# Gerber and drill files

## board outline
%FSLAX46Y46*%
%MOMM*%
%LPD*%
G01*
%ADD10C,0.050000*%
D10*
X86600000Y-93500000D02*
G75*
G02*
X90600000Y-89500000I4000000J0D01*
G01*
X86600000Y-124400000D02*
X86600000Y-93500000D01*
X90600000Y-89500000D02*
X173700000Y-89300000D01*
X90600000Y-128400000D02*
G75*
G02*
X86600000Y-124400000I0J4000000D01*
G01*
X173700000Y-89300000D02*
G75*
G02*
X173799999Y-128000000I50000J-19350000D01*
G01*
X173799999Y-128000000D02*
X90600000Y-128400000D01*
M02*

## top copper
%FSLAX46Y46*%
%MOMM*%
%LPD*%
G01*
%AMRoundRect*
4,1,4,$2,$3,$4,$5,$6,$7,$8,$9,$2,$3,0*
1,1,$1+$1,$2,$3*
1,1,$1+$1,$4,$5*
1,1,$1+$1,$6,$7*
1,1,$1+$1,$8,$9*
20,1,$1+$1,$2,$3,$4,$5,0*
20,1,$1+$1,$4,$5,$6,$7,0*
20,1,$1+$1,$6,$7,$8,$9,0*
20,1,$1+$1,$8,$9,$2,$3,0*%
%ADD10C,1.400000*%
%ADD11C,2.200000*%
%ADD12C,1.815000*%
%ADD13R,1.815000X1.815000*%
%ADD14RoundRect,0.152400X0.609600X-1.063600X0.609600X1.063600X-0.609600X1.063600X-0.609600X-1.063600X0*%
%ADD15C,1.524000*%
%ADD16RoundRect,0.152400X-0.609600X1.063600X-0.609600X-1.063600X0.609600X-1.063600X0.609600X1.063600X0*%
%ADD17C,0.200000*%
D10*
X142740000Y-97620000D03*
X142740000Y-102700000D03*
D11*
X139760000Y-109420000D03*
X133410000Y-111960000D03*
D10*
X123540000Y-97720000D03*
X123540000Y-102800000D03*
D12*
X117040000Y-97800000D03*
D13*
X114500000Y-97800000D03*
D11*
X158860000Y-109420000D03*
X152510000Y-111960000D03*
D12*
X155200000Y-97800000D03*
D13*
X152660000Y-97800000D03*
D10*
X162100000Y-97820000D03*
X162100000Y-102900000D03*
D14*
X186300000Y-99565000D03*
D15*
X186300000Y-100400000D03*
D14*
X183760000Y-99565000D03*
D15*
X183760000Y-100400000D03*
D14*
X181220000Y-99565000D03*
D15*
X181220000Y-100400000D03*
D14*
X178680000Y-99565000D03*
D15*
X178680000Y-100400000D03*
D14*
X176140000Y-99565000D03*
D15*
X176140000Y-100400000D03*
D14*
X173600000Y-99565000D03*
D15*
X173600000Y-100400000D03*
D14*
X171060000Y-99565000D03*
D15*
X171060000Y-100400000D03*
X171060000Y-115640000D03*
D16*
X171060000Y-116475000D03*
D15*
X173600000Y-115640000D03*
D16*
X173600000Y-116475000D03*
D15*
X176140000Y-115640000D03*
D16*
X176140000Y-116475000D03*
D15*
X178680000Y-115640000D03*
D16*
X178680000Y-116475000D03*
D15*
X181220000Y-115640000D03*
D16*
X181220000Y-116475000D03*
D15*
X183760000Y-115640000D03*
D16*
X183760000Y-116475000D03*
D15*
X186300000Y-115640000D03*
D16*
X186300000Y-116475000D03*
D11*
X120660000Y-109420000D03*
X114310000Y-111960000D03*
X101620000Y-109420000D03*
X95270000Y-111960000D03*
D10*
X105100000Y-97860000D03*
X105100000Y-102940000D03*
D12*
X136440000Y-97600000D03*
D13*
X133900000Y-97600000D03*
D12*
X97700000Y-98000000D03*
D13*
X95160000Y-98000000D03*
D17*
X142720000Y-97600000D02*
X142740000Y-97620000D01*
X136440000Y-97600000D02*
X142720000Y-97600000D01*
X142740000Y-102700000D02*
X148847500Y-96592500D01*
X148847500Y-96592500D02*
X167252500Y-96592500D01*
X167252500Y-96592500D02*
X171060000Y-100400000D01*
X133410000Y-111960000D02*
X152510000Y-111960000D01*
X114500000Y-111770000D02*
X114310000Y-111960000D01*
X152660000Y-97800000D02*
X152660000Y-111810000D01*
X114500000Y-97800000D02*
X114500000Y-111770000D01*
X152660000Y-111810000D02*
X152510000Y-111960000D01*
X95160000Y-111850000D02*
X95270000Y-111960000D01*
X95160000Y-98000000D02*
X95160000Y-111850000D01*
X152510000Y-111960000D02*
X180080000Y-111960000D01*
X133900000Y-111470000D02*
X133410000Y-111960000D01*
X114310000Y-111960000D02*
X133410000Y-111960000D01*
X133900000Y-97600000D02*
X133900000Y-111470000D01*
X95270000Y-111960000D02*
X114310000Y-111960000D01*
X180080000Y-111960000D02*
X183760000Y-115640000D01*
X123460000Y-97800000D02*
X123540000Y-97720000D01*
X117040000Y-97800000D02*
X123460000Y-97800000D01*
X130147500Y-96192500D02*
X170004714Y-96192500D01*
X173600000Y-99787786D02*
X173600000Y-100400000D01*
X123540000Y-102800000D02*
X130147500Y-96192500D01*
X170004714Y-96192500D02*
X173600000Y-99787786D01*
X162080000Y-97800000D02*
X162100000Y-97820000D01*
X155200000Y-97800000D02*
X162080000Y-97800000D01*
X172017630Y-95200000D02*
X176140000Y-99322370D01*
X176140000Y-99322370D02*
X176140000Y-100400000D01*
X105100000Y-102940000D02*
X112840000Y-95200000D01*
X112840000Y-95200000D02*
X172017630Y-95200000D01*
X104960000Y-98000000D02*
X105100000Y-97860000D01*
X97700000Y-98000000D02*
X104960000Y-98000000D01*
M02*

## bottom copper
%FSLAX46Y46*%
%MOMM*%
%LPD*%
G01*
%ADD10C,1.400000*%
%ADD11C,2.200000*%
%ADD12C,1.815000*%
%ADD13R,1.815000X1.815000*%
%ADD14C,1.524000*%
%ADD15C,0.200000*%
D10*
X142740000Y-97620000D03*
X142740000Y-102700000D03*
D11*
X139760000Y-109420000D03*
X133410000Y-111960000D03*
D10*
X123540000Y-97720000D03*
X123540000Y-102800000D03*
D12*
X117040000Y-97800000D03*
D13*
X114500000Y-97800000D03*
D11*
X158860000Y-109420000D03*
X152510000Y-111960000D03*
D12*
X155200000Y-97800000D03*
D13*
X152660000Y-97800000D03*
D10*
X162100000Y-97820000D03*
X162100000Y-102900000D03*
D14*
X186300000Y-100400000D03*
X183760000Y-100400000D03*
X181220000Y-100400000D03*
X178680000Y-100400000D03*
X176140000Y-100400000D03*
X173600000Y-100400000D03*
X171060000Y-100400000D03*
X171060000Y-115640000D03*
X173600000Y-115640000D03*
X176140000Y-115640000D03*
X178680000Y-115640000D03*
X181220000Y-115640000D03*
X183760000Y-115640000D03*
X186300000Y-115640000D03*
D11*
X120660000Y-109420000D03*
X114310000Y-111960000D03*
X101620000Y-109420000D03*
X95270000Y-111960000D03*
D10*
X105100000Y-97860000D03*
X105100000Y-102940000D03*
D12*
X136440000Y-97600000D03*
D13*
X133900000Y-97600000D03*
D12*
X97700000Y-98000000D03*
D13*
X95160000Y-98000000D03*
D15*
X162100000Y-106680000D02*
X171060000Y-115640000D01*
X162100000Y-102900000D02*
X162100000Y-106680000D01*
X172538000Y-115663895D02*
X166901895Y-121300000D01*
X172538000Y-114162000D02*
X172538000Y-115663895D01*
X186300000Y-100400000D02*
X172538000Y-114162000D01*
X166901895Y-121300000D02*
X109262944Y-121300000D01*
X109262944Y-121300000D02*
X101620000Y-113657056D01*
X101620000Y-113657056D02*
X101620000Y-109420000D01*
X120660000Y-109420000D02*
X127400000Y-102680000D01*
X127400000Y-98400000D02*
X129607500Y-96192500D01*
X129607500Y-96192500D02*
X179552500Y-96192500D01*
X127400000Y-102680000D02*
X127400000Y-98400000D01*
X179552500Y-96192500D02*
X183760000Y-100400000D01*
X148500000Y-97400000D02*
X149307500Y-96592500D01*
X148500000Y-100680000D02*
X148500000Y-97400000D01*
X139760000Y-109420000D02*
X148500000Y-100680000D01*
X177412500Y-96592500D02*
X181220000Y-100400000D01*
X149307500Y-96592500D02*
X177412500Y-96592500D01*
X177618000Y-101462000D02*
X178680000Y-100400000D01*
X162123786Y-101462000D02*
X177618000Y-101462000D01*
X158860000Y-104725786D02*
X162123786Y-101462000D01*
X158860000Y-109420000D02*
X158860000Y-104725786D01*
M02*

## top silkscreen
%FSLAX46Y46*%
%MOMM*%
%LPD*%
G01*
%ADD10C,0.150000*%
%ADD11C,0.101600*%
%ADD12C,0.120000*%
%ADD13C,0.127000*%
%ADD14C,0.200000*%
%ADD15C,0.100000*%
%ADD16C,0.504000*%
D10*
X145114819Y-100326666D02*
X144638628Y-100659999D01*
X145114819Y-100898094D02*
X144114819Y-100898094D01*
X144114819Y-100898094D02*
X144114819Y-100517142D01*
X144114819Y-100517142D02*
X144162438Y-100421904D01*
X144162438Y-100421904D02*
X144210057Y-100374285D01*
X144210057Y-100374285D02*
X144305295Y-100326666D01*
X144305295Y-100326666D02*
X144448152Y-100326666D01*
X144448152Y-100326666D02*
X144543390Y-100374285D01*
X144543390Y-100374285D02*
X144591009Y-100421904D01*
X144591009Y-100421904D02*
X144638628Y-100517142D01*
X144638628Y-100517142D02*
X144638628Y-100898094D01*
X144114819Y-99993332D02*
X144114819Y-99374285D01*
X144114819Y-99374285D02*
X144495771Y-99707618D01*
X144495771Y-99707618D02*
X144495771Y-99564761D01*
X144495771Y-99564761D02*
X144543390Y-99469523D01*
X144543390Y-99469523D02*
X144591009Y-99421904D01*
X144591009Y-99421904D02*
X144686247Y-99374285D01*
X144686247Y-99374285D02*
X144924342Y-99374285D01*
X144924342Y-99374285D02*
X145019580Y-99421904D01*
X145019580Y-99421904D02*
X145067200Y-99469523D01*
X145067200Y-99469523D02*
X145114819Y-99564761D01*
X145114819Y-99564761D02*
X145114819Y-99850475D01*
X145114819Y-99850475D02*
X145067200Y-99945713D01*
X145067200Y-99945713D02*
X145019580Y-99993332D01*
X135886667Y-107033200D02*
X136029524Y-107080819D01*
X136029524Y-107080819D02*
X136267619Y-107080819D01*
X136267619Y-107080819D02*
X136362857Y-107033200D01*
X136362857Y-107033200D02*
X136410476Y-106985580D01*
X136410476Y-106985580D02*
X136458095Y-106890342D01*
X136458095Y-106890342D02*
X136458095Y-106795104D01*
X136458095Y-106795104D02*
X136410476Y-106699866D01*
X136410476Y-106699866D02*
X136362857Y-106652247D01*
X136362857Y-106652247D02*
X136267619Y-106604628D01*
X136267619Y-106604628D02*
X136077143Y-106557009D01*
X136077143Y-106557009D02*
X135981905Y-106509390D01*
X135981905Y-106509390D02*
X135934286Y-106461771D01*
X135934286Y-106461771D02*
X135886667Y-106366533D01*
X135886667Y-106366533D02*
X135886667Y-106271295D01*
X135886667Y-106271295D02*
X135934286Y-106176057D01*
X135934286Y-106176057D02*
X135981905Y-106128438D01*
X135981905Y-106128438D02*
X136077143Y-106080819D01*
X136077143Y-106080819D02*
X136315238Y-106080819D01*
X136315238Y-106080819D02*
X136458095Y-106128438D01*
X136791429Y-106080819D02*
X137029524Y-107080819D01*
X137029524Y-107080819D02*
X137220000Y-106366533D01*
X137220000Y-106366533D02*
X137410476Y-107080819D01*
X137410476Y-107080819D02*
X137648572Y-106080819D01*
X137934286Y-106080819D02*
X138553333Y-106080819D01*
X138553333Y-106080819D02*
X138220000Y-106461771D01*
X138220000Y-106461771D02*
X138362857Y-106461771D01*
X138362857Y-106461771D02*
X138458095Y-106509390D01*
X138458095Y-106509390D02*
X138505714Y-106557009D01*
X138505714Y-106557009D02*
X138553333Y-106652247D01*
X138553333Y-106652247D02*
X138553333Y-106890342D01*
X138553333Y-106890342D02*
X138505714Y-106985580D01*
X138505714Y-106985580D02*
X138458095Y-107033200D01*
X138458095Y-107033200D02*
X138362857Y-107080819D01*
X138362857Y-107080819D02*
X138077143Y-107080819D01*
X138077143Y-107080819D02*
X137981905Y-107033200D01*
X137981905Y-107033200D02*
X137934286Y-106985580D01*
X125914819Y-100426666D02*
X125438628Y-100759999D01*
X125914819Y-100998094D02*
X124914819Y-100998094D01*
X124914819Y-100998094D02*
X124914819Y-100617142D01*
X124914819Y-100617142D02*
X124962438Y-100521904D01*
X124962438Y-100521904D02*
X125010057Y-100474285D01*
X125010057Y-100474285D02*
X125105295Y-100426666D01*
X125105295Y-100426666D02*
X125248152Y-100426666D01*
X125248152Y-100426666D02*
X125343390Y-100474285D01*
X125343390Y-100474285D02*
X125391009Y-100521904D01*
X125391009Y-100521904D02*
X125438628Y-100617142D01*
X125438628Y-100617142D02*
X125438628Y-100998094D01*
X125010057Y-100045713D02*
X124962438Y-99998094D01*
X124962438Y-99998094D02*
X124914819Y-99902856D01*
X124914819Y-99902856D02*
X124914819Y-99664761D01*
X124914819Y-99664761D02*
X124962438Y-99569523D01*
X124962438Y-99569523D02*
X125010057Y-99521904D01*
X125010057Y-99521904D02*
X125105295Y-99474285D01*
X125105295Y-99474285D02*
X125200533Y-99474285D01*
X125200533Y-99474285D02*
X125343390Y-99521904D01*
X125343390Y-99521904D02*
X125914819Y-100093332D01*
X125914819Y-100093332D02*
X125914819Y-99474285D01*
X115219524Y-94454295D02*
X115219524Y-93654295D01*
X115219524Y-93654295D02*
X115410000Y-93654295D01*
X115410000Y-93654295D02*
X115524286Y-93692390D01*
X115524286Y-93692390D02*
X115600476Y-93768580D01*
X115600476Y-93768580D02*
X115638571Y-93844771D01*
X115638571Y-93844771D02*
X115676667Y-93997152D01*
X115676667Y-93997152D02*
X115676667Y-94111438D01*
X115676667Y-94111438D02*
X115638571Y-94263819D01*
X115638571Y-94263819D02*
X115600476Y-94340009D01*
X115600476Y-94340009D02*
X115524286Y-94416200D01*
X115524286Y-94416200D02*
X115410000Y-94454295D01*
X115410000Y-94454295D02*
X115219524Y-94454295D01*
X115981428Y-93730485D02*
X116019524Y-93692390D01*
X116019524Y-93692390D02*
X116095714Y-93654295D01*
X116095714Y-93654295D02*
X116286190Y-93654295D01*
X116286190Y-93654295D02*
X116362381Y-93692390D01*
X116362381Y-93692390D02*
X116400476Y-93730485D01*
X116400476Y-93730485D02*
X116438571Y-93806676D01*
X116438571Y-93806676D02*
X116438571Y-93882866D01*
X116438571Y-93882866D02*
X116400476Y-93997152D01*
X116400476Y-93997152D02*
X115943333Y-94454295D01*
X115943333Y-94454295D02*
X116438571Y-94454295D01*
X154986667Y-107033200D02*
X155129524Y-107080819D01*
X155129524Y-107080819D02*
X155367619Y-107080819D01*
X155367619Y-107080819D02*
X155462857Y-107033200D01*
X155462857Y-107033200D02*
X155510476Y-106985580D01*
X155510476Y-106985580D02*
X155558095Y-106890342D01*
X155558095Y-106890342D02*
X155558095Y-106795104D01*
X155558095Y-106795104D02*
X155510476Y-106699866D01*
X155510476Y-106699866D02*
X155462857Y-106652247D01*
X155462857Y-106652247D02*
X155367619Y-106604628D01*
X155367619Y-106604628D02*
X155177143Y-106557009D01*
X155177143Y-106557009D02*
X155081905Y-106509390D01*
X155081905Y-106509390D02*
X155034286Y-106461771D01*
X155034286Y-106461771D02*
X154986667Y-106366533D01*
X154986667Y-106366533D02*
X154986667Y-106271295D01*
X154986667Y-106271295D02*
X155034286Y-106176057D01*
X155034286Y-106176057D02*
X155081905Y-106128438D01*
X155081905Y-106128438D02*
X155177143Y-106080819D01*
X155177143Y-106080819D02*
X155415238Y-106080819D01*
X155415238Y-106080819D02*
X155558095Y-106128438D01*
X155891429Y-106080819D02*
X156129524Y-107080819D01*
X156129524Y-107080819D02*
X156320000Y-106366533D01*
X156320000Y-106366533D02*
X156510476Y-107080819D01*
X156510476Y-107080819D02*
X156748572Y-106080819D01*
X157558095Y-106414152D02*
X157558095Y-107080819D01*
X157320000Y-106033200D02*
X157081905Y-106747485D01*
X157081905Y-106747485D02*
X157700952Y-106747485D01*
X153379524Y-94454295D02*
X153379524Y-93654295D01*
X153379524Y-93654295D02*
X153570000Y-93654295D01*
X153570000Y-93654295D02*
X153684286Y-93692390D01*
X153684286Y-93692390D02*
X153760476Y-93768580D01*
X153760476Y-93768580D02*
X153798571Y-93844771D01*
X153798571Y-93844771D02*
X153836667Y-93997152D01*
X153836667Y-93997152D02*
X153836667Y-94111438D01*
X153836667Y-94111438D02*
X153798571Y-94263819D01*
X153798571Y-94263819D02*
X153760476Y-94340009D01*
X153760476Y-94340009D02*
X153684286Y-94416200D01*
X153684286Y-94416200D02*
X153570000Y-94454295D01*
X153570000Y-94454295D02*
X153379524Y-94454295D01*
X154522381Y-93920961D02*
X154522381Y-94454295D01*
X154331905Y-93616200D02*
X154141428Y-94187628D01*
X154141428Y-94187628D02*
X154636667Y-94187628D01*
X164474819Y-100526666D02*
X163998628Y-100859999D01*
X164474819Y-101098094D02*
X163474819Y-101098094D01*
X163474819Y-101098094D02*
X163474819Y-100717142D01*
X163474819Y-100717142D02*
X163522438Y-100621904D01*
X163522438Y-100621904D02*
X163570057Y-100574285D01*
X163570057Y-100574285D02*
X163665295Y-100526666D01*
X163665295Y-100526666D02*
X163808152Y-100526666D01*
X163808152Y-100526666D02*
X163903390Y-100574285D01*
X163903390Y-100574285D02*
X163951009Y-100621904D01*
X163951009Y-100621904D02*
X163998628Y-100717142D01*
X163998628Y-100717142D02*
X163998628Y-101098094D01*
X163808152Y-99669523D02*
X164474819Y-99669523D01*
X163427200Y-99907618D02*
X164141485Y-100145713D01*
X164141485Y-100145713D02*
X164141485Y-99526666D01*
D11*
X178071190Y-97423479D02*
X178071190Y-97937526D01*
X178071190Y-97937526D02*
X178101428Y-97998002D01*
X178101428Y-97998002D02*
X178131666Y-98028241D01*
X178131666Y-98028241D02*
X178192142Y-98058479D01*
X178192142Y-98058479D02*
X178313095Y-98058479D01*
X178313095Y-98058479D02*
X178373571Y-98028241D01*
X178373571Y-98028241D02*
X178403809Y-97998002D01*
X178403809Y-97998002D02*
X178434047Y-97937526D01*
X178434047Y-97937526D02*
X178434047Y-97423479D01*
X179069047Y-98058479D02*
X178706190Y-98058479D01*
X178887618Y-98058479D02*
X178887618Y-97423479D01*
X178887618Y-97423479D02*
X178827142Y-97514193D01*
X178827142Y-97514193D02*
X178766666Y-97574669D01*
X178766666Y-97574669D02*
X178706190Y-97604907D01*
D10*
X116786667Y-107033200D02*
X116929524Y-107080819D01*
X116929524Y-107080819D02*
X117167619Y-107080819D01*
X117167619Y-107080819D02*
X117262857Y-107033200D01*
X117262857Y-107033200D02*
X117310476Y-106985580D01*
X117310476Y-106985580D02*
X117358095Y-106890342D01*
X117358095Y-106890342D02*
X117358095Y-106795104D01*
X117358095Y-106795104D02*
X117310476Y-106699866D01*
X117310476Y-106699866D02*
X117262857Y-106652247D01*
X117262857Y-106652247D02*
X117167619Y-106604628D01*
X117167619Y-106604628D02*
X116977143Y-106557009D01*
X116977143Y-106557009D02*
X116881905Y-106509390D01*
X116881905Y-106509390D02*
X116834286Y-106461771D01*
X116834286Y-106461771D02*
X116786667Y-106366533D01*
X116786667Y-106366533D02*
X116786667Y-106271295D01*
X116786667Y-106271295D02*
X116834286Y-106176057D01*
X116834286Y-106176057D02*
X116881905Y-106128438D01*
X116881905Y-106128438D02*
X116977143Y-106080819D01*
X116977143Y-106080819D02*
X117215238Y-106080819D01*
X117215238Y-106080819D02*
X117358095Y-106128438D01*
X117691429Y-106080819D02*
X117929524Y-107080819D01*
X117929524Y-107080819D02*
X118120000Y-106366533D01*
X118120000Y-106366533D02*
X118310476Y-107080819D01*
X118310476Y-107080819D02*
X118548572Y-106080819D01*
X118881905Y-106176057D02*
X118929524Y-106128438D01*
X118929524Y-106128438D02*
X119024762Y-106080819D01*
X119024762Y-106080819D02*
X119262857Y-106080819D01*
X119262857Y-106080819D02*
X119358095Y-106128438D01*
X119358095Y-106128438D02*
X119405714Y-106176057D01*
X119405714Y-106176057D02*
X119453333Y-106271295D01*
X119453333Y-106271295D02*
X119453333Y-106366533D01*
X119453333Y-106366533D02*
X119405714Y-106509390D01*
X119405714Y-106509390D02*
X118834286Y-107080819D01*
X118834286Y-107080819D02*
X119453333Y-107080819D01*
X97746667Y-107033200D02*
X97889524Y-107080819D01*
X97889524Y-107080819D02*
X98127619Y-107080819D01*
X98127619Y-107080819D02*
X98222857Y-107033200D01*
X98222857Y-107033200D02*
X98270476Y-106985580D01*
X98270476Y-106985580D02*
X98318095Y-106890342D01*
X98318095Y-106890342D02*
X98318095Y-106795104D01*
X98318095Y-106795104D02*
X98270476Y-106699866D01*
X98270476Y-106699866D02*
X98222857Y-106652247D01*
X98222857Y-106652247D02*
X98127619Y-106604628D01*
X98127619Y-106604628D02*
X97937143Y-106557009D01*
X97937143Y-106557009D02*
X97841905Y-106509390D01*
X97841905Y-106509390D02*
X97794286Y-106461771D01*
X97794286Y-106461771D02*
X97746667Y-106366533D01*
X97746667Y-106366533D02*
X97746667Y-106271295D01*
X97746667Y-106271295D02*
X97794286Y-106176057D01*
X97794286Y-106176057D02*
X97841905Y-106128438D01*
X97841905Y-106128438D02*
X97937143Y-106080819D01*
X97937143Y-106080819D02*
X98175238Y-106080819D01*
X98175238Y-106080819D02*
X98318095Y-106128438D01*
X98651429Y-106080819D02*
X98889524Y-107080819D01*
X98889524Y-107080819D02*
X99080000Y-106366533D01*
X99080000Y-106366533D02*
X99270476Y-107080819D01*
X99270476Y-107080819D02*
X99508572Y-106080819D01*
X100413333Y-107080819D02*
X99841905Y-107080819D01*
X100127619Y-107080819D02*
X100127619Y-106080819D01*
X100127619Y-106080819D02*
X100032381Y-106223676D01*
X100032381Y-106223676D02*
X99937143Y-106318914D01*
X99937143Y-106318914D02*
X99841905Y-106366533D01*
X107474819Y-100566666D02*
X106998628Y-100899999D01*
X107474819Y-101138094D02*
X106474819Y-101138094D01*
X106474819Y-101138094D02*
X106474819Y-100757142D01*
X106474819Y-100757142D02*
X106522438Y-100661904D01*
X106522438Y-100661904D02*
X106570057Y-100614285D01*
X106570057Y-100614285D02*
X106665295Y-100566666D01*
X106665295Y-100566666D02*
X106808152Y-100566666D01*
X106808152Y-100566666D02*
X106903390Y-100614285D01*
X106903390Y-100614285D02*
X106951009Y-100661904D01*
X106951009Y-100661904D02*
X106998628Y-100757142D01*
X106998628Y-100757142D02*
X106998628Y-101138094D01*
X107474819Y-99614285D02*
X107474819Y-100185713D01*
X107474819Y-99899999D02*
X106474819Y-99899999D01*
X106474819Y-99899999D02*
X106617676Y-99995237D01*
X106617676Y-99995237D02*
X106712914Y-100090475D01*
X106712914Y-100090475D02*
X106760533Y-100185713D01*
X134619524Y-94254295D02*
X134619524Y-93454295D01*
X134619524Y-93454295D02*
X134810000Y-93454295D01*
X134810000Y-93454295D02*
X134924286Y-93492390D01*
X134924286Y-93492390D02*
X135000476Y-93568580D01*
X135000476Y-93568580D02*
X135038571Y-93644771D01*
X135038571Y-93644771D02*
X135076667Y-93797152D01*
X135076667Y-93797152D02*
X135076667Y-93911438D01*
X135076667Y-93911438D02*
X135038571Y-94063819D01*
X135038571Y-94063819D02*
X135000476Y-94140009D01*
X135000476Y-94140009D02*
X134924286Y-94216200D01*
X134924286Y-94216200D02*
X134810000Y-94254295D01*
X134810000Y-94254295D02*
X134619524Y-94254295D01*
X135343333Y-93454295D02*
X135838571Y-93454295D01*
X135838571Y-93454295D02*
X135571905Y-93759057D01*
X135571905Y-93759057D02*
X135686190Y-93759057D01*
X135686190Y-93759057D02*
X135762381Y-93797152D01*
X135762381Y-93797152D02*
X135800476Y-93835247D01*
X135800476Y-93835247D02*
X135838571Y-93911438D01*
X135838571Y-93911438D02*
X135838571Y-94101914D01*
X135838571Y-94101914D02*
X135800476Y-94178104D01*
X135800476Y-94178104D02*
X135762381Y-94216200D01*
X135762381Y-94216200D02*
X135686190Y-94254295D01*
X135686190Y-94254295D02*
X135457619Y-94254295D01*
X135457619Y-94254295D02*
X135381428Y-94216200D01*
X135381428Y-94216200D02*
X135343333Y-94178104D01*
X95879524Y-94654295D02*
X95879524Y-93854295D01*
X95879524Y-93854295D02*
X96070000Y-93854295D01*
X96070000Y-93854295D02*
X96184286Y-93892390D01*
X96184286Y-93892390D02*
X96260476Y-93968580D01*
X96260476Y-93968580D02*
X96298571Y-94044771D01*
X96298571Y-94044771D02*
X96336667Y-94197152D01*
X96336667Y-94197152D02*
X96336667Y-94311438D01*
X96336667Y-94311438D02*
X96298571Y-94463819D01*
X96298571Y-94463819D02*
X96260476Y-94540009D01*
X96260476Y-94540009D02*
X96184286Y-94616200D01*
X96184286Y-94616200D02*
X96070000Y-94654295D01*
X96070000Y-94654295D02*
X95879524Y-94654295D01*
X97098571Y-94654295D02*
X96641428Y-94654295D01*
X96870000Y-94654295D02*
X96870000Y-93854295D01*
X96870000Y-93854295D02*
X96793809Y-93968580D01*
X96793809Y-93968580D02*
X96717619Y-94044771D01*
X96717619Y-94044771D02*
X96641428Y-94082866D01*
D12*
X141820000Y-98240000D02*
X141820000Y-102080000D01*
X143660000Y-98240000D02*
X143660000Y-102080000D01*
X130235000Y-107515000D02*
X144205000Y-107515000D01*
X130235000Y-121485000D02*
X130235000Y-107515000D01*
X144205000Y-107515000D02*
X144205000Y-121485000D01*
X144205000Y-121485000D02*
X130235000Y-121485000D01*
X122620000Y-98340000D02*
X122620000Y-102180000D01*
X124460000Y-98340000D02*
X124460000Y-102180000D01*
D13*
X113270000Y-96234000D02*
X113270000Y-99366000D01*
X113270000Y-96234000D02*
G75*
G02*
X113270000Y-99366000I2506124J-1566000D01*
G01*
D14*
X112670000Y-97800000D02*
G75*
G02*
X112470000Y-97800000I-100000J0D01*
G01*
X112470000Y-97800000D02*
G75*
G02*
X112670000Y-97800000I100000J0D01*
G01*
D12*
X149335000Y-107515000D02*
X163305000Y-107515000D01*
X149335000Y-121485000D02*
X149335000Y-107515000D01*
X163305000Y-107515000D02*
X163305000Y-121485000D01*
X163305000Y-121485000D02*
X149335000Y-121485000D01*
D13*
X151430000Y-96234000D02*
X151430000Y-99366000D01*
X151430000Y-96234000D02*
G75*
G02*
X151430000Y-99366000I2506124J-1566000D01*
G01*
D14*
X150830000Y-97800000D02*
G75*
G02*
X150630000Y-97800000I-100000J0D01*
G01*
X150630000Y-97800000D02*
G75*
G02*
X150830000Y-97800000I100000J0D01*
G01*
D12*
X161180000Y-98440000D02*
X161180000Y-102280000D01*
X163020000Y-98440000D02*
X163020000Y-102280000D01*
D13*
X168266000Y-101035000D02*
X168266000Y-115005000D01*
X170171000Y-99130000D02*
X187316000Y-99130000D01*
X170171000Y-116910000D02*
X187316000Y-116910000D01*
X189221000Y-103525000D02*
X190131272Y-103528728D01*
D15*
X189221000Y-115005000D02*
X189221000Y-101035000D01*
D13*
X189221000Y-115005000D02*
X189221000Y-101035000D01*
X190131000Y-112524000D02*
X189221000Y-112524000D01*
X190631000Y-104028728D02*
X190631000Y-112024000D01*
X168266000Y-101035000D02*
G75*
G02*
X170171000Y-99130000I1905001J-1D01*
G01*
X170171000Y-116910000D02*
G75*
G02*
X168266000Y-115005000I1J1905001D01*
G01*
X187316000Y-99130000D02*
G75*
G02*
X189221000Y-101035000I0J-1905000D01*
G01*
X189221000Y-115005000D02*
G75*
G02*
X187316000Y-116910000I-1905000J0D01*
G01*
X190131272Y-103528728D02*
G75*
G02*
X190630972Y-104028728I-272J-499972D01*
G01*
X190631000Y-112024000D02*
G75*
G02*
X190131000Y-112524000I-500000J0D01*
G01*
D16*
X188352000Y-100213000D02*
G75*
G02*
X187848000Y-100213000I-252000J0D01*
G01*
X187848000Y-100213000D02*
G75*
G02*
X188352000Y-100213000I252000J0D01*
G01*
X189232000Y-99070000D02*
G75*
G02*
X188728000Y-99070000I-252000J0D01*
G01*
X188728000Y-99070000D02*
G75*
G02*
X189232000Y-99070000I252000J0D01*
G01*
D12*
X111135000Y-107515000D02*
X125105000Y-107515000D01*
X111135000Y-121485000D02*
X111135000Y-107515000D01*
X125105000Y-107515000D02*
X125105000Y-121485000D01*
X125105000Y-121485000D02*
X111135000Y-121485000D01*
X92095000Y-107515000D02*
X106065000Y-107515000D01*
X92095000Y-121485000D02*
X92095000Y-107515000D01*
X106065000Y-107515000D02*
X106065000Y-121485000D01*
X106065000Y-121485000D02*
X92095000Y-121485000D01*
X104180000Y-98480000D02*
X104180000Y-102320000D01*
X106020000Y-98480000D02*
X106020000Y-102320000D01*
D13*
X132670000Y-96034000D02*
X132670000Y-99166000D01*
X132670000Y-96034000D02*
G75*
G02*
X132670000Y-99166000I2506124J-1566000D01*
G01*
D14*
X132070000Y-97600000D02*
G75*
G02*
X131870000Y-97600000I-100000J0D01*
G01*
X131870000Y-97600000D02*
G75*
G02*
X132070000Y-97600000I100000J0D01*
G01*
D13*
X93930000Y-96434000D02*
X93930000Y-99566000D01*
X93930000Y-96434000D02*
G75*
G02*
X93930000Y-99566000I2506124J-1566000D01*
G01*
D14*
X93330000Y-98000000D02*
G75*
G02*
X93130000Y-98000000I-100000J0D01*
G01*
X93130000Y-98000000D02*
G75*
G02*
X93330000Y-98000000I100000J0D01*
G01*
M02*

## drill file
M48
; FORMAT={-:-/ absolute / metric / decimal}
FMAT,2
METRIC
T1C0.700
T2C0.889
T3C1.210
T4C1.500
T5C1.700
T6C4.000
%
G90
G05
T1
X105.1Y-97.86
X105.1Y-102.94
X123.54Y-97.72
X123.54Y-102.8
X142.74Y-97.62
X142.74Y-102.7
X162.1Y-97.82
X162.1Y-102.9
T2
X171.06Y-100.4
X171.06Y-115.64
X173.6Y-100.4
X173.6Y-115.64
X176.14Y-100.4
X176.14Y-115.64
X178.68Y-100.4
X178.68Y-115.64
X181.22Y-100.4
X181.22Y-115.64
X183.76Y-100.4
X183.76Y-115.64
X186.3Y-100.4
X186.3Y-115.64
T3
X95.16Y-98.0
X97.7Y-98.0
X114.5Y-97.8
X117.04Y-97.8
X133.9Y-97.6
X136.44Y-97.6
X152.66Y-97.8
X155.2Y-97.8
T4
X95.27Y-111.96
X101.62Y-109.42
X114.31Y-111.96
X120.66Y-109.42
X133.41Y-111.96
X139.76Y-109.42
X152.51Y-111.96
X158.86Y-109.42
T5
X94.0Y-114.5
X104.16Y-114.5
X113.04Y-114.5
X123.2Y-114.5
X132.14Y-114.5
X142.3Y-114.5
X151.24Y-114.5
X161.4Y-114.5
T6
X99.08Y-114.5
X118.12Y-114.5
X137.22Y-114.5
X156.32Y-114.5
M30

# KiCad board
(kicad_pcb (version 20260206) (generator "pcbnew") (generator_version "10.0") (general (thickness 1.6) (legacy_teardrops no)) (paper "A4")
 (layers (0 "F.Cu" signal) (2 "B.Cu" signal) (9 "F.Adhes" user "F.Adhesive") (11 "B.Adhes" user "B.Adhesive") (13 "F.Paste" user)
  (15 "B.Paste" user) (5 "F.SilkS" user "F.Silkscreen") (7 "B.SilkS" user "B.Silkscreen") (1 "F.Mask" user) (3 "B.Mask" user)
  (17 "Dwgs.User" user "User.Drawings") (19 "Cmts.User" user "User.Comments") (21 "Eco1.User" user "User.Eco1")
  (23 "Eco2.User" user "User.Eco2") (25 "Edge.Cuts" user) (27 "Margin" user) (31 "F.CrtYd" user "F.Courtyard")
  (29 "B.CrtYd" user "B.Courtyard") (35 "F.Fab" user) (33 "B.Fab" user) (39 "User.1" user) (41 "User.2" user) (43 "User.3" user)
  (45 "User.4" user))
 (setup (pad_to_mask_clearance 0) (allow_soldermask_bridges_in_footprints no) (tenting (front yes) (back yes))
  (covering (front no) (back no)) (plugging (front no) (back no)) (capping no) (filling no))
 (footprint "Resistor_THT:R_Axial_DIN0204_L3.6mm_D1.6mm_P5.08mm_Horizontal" (layer "F.Cu") (at 142.74 97.62 -90)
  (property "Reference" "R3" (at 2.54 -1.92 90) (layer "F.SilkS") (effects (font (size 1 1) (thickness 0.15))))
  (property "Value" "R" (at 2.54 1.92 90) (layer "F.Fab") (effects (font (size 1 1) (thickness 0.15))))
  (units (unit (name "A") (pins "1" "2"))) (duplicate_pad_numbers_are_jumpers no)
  (fp_line (start 0.62 0.92) (end 4.46 0.92) (stroke (width 0.12) (type solid)) (layer "F.SilkS"))
  (fp_line (start 0.62 -0.92) (end 4.46 -0.92) (stroke (width 0.12) (type solid)) (layer "F.SilkS"))
  (pad "1" thru_hole circle (at 0 0 270) (size 1.4 1.4) (drill 0.7) (layers "*.Cu" "*.Mask") (remove_unused_layers no) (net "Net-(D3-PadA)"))
  (pad "2" thru_hole circle (at 5.08 0 270) (size 1.4 1.4) (drill 0.7) (layers "*.Cu" "*.Mask") (remove_unused_layers no) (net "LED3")))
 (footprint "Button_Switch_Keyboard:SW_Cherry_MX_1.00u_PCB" (layer "F.Cu") (at 139.76 109.42)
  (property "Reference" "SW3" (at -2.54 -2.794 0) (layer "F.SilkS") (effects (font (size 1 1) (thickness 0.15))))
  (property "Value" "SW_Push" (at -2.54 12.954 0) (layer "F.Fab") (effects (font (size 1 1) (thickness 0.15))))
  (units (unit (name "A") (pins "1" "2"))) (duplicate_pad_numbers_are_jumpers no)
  (fp_line (start -9.525 -1.905) (end 4.445 -1.905) (stroke (width 0.12) (type solid)) (layer "F.SilkS"))
  (fp_line (start -9.525 12.065) (end -9.525 -1.905) (stroke (width 0.12) (type solid)) (layer "F.SilkS"))
  (fp_line (start 4.445 -1.905) (end 4.445 12.065) (stroke (width 0.12) (type solid)) (layer "F.SilkS"))
  (fp_line (start 4.445 12.065) (end -9.525 12.065) (stroke (width 0.12) (type solid)) (layer "F.SilkS"))
  (pad "" np_thru_hole circle (at -7.62 5.08) (size 1.7 1.7) (drill 1.7) (layers "*.Cu" "*.Mask"))
  (pad "" np_thru_hole circle (at -2.54 5.08) (size 4 4) (drill 4) (layers "*.Cu" "*.Mask"))
  (pad "" np_thru_hole circle (at 2.54 5.08) (size 1.7 1.7) (drill 1.7) (layers "*.Cu" "*.Mask"))
  (pad "1" thru_hole circle (at 0 0) (size 2.2 2.2) (drill 1.5) (layers "*.Cu" "*.Mask") (remove_unused_layers no) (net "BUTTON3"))
  (pad "2" thru_hole circle (at -6.35 2.54) (size 2.2 2.2) (drill 1.5) (layers "*.Cu" "*.Mask") (remove_unused_layers no) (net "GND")))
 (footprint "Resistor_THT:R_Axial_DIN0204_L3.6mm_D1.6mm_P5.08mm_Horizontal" (layer "F.Cu") (at 123.54 97.72 -90)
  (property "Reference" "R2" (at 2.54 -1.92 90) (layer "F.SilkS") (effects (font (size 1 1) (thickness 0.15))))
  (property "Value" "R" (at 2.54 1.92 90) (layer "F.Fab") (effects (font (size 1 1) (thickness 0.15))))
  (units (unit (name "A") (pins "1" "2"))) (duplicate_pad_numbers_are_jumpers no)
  (fp_line (start 0.62 0.92) (end 4.46 0.92) (stroke (width 0.12) (type solid)) (layer "F.SilkS"))
  (fp_line (start 0.62 -0.92) (end 4.46 -0.92) (stroke (width 0.12) (type solid)) (layer "F.SilkS"))
  (pad "1" thru_hole circle (at 0 0 270) (size 1.4 1.4) (drill 0.7) (layers "*.Cu" "*.Mask") (remove_unused_layers no) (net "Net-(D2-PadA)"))
  (pad "2" thru_hole circle (at 5.08 0 270) (size 1.4 1.4) (drill 0.7) (layers "*.Cu" "*.Mask") (remove_unused_layers no) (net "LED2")))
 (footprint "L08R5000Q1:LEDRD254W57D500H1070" (layer "F.Cu") (at 115.77 97.8)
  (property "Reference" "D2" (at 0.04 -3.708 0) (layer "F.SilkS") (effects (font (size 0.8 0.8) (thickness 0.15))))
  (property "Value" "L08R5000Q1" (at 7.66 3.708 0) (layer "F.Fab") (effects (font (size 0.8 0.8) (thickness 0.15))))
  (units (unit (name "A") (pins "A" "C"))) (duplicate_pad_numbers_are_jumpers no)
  (fp_line (start -2.5 -1.566) (end -2.5 1.566) (stroke (width 0.127) (type solid)) (layer "F.SilkS"))
  (fp_arc (start -2.5 -1.566) (mid 2.961291 0) (end -2.5 1.566) (stroke (width 0.127) (type solid)) (layer "F.SilkS"))
  (fp_circle (center -3.2 0) (end -3.1 0) (stroke (width 0.2) (type solid)) (fill no) (layer "F.SilkS"))
  (pad "A" thru_hole circle (at 1.27 0) (size 1.815 1.815) (drill 1.21) (layers "*.Cu" "*.Mask") (remove_unused_layers no)
   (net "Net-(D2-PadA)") (solder_mask_margin 0.102))
  (pad "C" thru_hole rect (at -1.27 0) (size 1.815 1.815) (drill 1.21) (layers "*.Cu" "*.Mask") (remove_unused_layers no) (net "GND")
   (solder_mask_margin 0.102)))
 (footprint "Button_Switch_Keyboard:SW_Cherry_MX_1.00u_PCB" (layer "F.Cu") (at 158.86 109.42)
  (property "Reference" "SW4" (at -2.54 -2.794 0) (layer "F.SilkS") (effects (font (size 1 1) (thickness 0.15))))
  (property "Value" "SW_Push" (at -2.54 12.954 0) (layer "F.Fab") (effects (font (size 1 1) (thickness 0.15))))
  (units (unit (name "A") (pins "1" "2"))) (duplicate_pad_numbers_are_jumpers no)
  (fp_line (start -9.525 -1.905) (end 4.445 -1.905) (stroke (width 0.12) (type solid)) (layer "F.SilkS"))
  (fp_line (start -9.525 12.065) (end -9.525 -1.905) (stroke (width 0.12) (type solid)) (layer "F.SilkS"))
  (fp_line (start 4.445 -1.905) (end 4.445 12.065) (stroke (width 0.12) (type solid)) (layer "F.SilkS"))
  (fp_line (start 4.445 12.065) (end -9.525 12.065) (stroke (width 0.12) (type solid)) (layer "F.SilkS"))
  (pad "" np_thru_hole circle (at -7.62 5.08) (size 1.7 1.7) (drill 1.7) (layers "*.Cu" "*.Mask"))
  (pad "" np_thru_hole circle (at -2.54 5.08) (size 4 4) (drill 4) (layers "*.Cu" "*.Mask"))
  (pad "" np_thru_hole circle (at 2.54 5.08) (size 1.7 1.7) (drill 1.7) (layers "*.Cu" "*.Mask"))
  (pad "1" thru_hole circle (at 0 0) (size 2.2 2.2) (drill 1.5) (layers "*.Cu" "*.Mask") (remove_unused_layers no) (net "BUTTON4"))
  (pad "2" thru_hole circle (at -6.35 2.54) (size 2.2 2.2) (drill 1.5) (layers "*.Cu" "*.Mask") (remove_unused_layers no) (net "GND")))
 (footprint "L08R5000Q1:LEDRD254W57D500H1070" (layer "F.Cu") (at 153.93 97.8)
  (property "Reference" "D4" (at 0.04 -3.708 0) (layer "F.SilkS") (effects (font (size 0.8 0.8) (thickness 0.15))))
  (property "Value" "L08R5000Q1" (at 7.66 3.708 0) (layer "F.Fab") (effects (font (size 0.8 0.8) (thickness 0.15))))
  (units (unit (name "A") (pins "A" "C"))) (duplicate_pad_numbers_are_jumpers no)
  (fp_line (start -2.5 -1.566) (end -2.5 1.566) (stroke (width 0.127) (type solid)) (layer "F.SilkS"))
  (fp_arc (start -2.5 -1.566) (mid 2.961291 0) (end -2.5 1.566) (stroke (width 0.127) (type solid)) (layer "F.SilkS"))
  (fp_circle (center -3.2 0) (end -3.1 0) (stroke (width 0.2) (type solid)) (fill no) (layer "F.SilkS"))
  (pad "A" thru_hole circle (at 1.27 0) (size 1.815 1.815) (drill 1.21) (layers "*.Cu" "*.Mask") (remove_unused_layers no)
   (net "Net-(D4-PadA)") (solder_mask_margin 0.102))
  (pad "C" thru_hole rect (at -1.27 0) (size 1.815 1.815) (drill 1.21) (layers "*.Cu" "*.Mask") (remove_unused_layers no) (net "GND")
   (solder_mask_margin 0.102)))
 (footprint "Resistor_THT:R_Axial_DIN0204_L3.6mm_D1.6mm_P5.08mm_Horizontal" (layer "F.Cu") (at 162.1 97.82 -90)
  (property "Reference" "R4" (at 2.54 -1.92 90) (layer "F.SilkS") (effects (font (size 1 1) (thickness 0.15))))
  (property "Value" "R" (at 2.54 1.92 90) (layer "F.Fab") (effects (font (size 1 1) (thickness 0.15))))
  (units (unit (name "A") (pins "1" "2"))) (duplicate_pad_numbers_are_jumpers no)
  (fp_line (start 0.62 0.92) (end 4.46 0.92) (stroke (width 0.12) (type solid)) (layer "F.SilkS"))
  (fp_line (start 0.62 -0.92) (end 4.46 -0.92) (stroke (width 0.12) (type solid)) (layer "F.SilkS"))
  (pad "1" thru_hole circle (at 0 0 270) (size 1.4 1.4) (drill 0.7) (layers "*.Cu" "*.Mask") (remove_unused_layers no) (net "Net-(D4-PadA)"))
  (pad "2" thru_hole circle (at 5.08 0 270) (size 1.4 1.4) (drill 0.7) (layers "*.Cu" "*.Mask") (remove_unused_layers no) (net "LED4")))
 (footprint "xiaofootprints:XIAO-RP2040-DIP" (layer "F.Cu") (at 178.68 108.02)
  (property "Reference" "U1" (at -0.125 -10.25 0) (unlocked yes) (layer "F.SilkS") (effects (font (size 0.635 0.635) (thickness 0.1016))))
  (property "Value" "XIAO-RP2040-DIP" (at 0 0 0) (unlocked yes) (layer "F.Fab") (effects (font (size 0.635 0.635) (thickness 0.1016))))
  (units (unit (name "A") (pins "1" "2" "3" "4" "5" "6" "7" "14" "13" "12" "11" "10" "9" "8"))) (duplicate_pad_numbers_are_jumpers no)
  (fp_line (start -10.414 -6.985) (end -10.414 6.985) (stroke (width 0.127) (type solid)) (layer "F.SilkS"))
  (fp_line (start -8.509 -8.89) (end 8.636 -8.89) (stroke (width 0.127) (type solid)) (layer "F.SilkS"))
  (fp_line (start -8.509 8.89) (end 8.636 8.89) (stroke (width 0.127) (type solid)) (layer "F.SilkS"))
  (fp_line (start 10.541 -4.495) (end 11.451272 -4.491272) (stroke (width 0.127) (type solid)) (layer "F.SilkS"))
  (fp_line (start 10.541 6.985) (end 10.541 -6.985) (stroke (width 0.1) (type solid)) (layer "F.SilkS"))
  (fp_line (start 10.541 6.985) (end 10.541 -6.985) (stroke (width 0.127) (type solid)) (layer "F.SilkS"))
  (fp_line (start 11.451 4.504) (end 10.541 4.504) (stroke (width 0.127) (type solid)) (layer "F.SilkS"))
  (fp_line (start 11.951 -3.991272) (end 11.951 4.004) (stroke (width 0.127) (type solid)) (layer "F.SilkS"))
  (fp_arc (start -10.414 -6.985) (mid -9.856038 -8.332038) (end -8.509 -8.89) (stroke (width 0.127) (type solid)) (layer "F.SilkS"))
  (fp_arc (start -8.509 8.89) (mid -9.856038 8.332038) (end -10.414 6.985) (stroke (width 0.127) (type solid)) (layer "F.SilkS"))
  (fp_arc (start 8.636 -8.89) (mid 9.983038 -8.332038) (end 10.541 -6.985) (stroke (width 0.127) (type solid)) (layer "F.SilkS"))
  (fp_arc (start 10.541 6.985) (mid 9.983038 8.332038) (end 8.636 8.89) (stroke (width 0.127) (type solid)) (layer "F.SilkS"))
  (fp_arc (start 11.451272 -4.491272) (mid 11.804644 -4.344724) (end 11.951 -3.991272) (stroke (width 0.127) (type default))
   (layer "F.SilkS"))
  (fp_arc (start 11.951 4.004) (mid 11.804553 4.357553) (end 11.451 4.504) (stroke (width 0.127) (type default)) (layer "F.SilkS"))
  (fp_circle (center 9.42 -7.807) (end 9.674 -7.807) (stroke (width 0.5) (type solid)) (fill yes) (layer "F.SilkS"))
  (fp_circle (center 10.3 -8.95) (end 10.554 -8.95) (stroke (width 0.5) (type solid)) (fill yes) (layer "F.SilkS"))
  (pad "1" smd roundrect (at 7.62 -8.455 90) (size 2.432 1.524) (layers "F.Cu" "F.Mask") (roundrect_rratio 0.1) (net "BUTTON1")
   (thermal_bridge_angle 45))
  (pad "1" thru_hole circle (at 7.62 -7.62 90) (size 1.524 1.524) (drill 0.889) (layers "*.Cu" "*.Mask") (remove_unused_layers no)
   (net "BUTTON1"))
  (pad "2" smd roundrect (at 5.08 -8.455 90) (size 2.432 1.524) (layers "F.Cu" "F.Mask") (roundrect_rratio 0.1) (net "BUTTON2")
   (thermal_bridge_angle 45))
  (pad "2" thru_hole circle (at 5.08 -7.62 90) (size 1.524 1.524) (drill 0.889) (layers "*.Cu" "*.Mask") (remove_unused_layers no)
   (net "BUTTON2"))
  (pad "3" smd roundrect (at 2.54 -8.455 90) (size 2.432 1.524) (layers "F.Cu" "F.Mask") (roundrect_rratio 0.1) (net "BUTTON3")
   (thermal_bridge_angle 45))
  (pad "3" thru_hole circle (at 2.54 -7.62 90) (size 1.524 1.524) (drill 0.889) (layers "*.Cu" "*.Mask") (remove_unused_layers no)
   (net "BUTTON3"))
  (pad "4" smd roundrect (at 0 -8.455 90) (size 2.432 1.524) (layers "F.Cu" "F.Mask") (roundrect_rratio 0.1) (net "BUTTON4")
   (thermal_bridge_angle 45))
  (pad "4" thru_hole circle (at 0 -7.62 90) (size 1.524 1.524) (drill 0.889) (layers "*.Cu" "*.Mask") (remove_unused_layers no)
   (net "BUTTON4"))
  (pad "5" smd roundrect (at -2.54 -8.455 90) (size 2.432 1.524) (layers "F.Cu" "F.Mask") (roundrect_rratio 0.1) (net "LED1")
   (thermal_bridge_angle 45))
  (pad "5" thru_hole circle (at -2.54 -7.62 90) (size 1.524 1.524) (drill 0.889) (layers "*.Cu" "*.Mask") (remove_unused_layers no)
   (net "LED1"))
  (pad "6" smd roundrect (at -5.08 -8.455 90) (size 2.432 1.524) (layers "F.Cu" "F.Mask") (roundrect_rratio 0.1) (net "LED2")
   (thermal_bridge_angle 45))
  (pad "6" thru_hole circle (at -5.08 -7.62 90) (size 1.524 1.524) (drill 0.889) (layers "*.Cu" "*.Mask") (remove_unused_layers no)
   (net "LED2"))
  (pad "7" smd roundrect (at -7.62 -8.455 90) (size 2.432 1.524) (layers "F.Cu" "F.Mask") (roundrect_rratio 0.1) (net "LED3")
   (thermal_bridge_angle 45))
  (pad "7" thru_hole circle (at -7.62 -7.62 90) (size 1.524 1.524) (drill 0.889) (layers "*.Cu" "*.Mask") (remove_unused_layers no)
   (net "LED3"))
  (pad "8" thru_hole circle (at -7.62 7.62 270) (size 1.524 1.524) (drill 0.889) (layers "*.Cu" "*.Mask") (remove_unused_layers no)
   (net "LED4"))
  (pad "8" smd roundrect (at -7.62 8.455 270) (size 2.432 1.524) (layers "F.Cu" "F.Mask") (roundrect_rratio 0.1) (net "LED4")
   (thermal_bridge_angle 45))
  (pad "9" thru_hole circle (at -5.08 7.62 270) (size 1.524 1.524) (drill 0.889) (layers "*.Cu" "*.Mask") (remove_unused_layers no)
   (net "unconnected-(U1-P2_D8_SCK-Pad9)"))
  (pad "9" smd roundrect (at -5.08 8.455 270) (size 2.432 1.524) (layers "F.Cu" "F.Mask") (roundrect_rratio 0.1)
   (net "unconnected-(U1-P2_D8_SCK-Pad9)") (thermal_bridge_angle 45))
  (pad "10" thru_hole circle (at -2.54 7.62 270) (size 1.524 1.524) (drill 0.889) (layers "*.Cu" "*.Mask") (remove_unused_layers no)
   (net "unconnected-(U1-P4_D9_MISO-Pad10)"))
  (pad "10" smd roundrect (at -2.54 8.455 270) (size 2.432 1.524) (layers "F.Cu" "F.Mask") (roundrect_rratio 0.1)
   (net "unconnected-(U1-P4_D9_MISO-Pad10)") (thermal_bridge_angle 45))
  (pad "11" thru_hole circle (at 0 7.62 270) (size 1.524 1.524) (drill 0.889) (layers "*.Cu" "*.Mask") (remove_unused_layers no)
   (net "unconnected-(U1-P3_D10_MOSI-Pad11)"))
  (pad "11" smd roundrect (at 0 8.455 270) (size 2.432 1.524) (layers "F.Cu" "F.Mask") (roundrect_rratio 0.1)
   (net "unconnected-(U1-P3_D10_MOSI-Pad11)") (thermal_bridge_angle 45))
  (pad "12" thru_hole circle (at 2.54 7.62 270) (size 1.524 1.524) (drill 0.889) (layers "*.Cu" "*.Mask") (remove_unused_layers no)
   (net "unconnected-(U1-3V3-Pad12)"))
  (pad "12" smd roundrect (at 2.54 8.455 270) (size 2.432 1.524) (layers "F.Cu" "F.Mask") (roundrect_rratio 0.1)
   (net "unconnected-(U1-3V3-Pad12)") (thermal_bridge_angle 45))
  (pad "13" thru_hole circle (at 5.08 7.62 270) (size 1.524 1.524) (drill 0.889) (layers "*.Cu" "*.Mask") (remove_unused_layers no)
   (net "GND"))
  (pad "13" smd roundrect (at 5.08 8.455 270) (size 2.432 1.524) (layers "F.Cu" "F.Mask") (roundrect_rratio 0.1) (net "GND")
   (thermal_bridge_angle 45))
  (pad "14" thru_hole circle (at 7.62 7.62 270) (size 1.524 1.524) (drill 0.889) (layers "*.Cu" "*.Mask") (remove_unused_layers no)
   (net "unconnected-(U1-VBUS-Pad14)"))
  (pad "14" smd roundrect (at 7.62 8.455 270) (size 2.432 1.524) (layers "F.Cu" "F.Mask") (roundrect_rratio 0.1)
   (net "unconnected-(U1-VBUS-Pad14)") (thermal_bridge_angle 45)))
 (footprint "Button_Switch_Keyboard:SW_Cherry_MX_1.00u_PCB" (layer "F.Cu") (at 120.66 109.42)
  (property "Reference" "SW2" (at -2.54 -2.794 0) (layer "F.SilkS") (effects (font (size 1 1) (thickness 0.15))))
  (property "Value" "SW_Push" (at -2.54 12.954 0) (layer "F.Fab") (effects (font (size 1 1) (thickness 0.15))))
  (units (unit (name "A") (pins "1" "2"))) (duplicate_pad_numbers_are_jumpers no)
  (fp_line (start -9.525 -1.905) (end 4.445 -1.905) (stroke (width 0.12) (type solid)) (layer "F.SilkS"))
  (fp_line (start -9.525 12.065) (end -9.525 -1.905) (stroke (width 0.12) (type solid)) (layer "F.SilkS"))
  (fp_line (start 4.445 -1.905) (end 4.445 12.065) (stroke (width 0.12) (type solid)) (layer "F.SilkS"))
  (fp_line (start 4.445 12.065) (end -9.525 12.065) (stroke (width 0.12) (type solid)) (layer "F.SilkS"))
  (pad "" np_thru_hole circle (at -7.62 5.08) (size 1.7 1.7) (drill 1.7) (layers "*.Cu" "*.Mask"))
  (pad "" np_thru_hole circle (at -2.54 5.08) (size 4 4) (drill 4) (layers "*.Cu" "*.Mask"))
  (pad "" np_thru_hole circle (at 2.54 5.08) (size 1.7 1.7) (drill 1.7) (layers "*.Cu" "*.Mask"))
  (pad "1" thru_hole circle (at 0 0) (size 2.2 2.2) (drill 1.5) (layers "*.Cu" "*.Mask") (remove_unused_layers no) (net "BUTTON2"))
  (pad "2" thru_hole circle (at -6.35 2.54) (size 2.2 2.2) (drill 1.5) (layers "*.Cu" "*.Mask") (remove_unused_layers no) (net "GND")))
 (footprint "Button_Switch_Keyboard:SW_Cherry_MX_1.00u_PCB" (layer "F.Cu") (at 101.62 109.42)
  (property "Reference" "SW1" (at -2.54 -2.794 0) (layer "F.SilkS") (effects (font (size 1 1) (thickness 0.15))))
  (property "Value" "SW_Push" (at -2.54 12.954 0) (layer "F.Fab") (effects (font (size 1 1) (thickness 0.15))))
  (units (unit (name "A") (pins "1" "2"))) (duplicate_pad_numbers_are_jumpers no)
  (fp_line (start -9.525 -1.905) (end 4.445 -1.905) (stroke (width 0.12) (type solid)) (layer "F.SilkS"))
  (fp_line (start -9.525 12.065) (end -9.525 -1.905) (stroke (width 0.12) (type solid)) (layer "F.SilkS"))
  (fp_line (start 4.445 -1.905) (end 4.445 12.065) (stroke (width 0.12) (type solid)) (layer "F.SilkS"))
  (fp_line (start 4.445 12.065) (end -9.525 12.065) (stroke (width 0.12) (type solid)) (layer "F.SilkS"))
  (pad "" np_thru_hole circle (at -7.62 5.08) (size 1.7 1.7) (drill 1.7) (layers "*.Cu" "*.Mask"))
  (pad "" np_thru_hole circle (at -2.54 5.08) (size 4 4) (drill 4) (layers "*.Cu" "*.Mask"))
  (pad "" np_thru_hole circle (at 2.54 5.08) (size 1.7 1.7) (drill 1.7) (layers "*.Cu" "*.Mask"))
  (pad "1" thru_hole circle (at 0 0) (size 2.2 2.2) (drill 1.5) (layers "*.Cu" "*.Mask") (remove_unused_layers no) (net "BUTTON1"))
  (pad "2" thru_hole circle (at -6.35 2.54) (size 2.2 2.2) (drill 1.5) (layers "*.Cu" "*.Mask") (remove_unused_layers no) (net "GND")))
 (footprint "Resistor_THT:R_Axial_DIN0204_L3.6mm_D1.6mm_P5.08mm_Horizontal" (layer "F.Cu") (at 105.1 97.86 -90)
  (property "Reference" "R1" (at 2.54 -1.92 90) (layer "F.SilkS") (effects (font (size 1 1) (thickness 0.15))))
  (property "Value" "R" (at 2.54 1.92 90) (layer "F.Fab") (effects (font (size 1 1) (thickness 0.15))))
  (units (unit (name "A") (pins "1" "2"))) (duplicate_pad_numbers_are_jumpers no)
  (fp_line (start 0.62 0.92) (end 4.46 0.92) (stroke (width 0.12) (type solid)) (layer "F.SilkS"))
  (fp_line (start 0.62 -0.92) (end 4.46 -0.92) (stroke (width 0.12) (type solid)) (layer "F.SilkS"))
  (pad "1" thru_hole circle (at 0 0 270) (size 1.4 1.4) (drill 0.7) (layers "*.Cu" "*.Mask") (remove_unused_layers no) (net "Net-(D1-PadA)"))
  (pad "2" thru_hole circle (at 5.08 0 270) (size 1.4 1.4) (drill 0.7) (layers "*.Cu" "*.Mask") (remove_unused_layers no) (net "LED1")))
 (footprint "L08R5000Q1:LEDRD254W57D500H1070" (layer "F.Cu") (at 135.17 97.6)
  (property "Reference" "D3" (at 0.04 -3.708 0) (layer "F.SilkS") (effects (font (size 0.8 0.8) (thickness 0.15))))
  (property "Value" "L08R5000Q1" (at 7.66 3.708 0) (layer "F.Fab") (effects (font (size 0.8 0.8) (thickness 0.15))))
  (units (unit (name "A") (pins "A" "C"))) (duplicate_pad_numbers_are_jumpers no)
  (fp_line (start -2.5 -1.566) (end -2.5 1.566) (stroke (width 0.127) (type solid)) (layer "F.SilkS"))
  (fp_arc (start -2.5 -1.566) (mid 2.961291 0) (end -2.5 1.566) (stroke (width 0.127) (type solid)) (layer "F.SilkS"))
  (fp_circle (center -3.2 0) (end -3.1 0) (stroke (width 0.2) (type solid)) (fill no) (layer "F.SilkS"))
  (pad "A" thru_hole circle (at 1.27 0) (size 1.815 1.815) (drill 1.21) (layers "*.Cu" "*.Mask") (remove_unused_layers no)
   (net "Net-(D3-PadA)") (solder_mask_margin 0.102))
  (pad "C" thru_hole rect (at -1.27 0) (size 1.815 1.815) (drill 1.21) (layers "*.Cu" "*.Mask") (remove_unused_layers no) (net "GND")
   (solder_mask_margin 0.102)))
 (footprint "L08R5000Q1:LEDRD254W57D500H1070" (layer "F.Cu") (at 96.43 98)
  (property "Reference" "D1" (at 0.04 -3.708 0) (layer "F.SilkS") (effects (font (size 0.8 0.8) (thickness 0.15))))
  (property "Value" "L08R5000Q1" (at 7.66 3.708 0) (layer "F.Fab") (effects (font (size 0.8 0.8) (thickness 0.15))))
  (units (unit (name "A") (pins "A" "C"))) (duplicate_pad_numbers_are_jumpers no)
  (fp_line (start -2.5 -1.566) (end -2.5 1.566) (stroke (width 0.127) (type solid)) (layer "F.SilkS"))
  (fp_arc (start -2.5 -1.566) (mid 2.961291 0) (end -2.5 1.566) (stroke (width 0.127) (type solid)) (layer "F.SilkS"))
  (fp_circle (center -3.2 0) (end -3.1 0) (stroke (width 0.2) (type solid)) (fill no) (layer "F.SilkS"))
  (pad "A" thru_hole circle (at 1.27 0) (size 1.815 1.815) (drill 1.21) (layers "*.Cu" "*.Mask") (remove_unused_layers no)
   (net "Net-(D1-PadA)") (solder_mask_margin 0.102))
  (pad "C" thru_hole rect (at -1.27 0) (size 1.815 1.815) (drill 1.21) (layers "*.Cu" "*.Mask") (remove_unused_layers no) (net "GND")
   (solder_mask_margin 0.102)))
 (gr_arc (start 86.6 93.5) (mid 87.771573 90.671573) (end 90.6 89.5) (stroke (width 0.05) (type solid)) (layer "Edge.Cuts"))
 (gr_line (start 86.6 124.4) (end 86.6 93.5) (stroke (width 0.05) (type default)) (layer "Edge.Cuts"))
 (gr_line (start 90.6 89.5) (end 173.7 89.3) (stroke (width 0.05) (type default)) (layer "Edge.Cuts"))
 (gr_arc (start 90.6 128.4) (mid 87.771573 127.228427) (end 86.6 124.4) (stroke (width 0.05) (type default)) (layer "Edge.Cuts"))
 (gr_arc (start 173.7 89.3) (mid 193.1 108.6) (end 173.799999 128) (stroke (width 0.05) (type default)) (layer "Edge.Cuts"))
 (gr_line (start 173.799999 128) (end 90.6 128.4) (stroke (width 0.05) (type default)) (layer "Edge.Cuts"))
 (segment (start 142.72 97.6) (end 142.74 97.62) (width 0.2) (layer "F.Cu") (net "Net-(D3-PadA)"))
 (segment (start 136.44 97.6) (end 142.72 97.6) (width 0.2) (layer "F.Cu") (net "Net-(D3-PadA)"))
 (segment (start 142.74 102.7) (end 148.8475 96.5925) (width 0.2) (layer "F.Cu") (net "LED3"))
 (segment (start 148.8475 96.5925) (end 167.2525 96.5925) (width 0.2) (layer "F.Cu") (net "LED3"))
 (segment (start 167.2525 96.5925) (end 171.06 100.4) (width 0.2) (layer "F.Cu") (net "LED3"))
 (segment (start 133.41 111.96) (end 152.51 111.96) (width 0.2) (layer "F.Cu") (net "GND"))
 (segment (start 114.5 111.77) (end 114.31 111.96) (width 0.2) (layer "F.Cu") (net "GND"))
 (segment (start 152.66 97.8) (end 152.66 111.81) (width 0.2) (layer "F.Cu") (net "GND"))
 (segment (start 114.5 97.8) (end 114.5 111.77) (width 0.2) (layer "F.Cu") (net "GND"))
 (segment (start 152.66 111.81) (end 152.51 111.96) (width 0.2) (layer "F.Cu") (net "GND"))
 (segment (start 95.16 111.85) (end 95.27 111.96) (width 0.2) (layer "F.Cu") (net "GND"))
 (segment (start 95.16 98) (end 95.16 111.85) (width 0.2) (layer "F.Cu") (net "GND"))
 (segment (start 152.51 111.96) (end 180.08 111.96) (width 0.2) (layer "F.Cu") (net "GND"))
 (segment (start 133.9 111.47) (end 133.41 111.96) (width 0.2) (layer "F.Cu") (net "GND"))
 (segment (start 114.31 111.96) (end 133.41 111.96) (width 0.2) (layer "F.Cu") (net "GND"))
 (segment (start 133.9 97.6) (end 133.9 111.47) (width 0.2) (layer "F.Cu") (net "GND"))
 (segment (start 95.27 111.96) (end 114.31 111.96) (width 0.2) (layer "F.Cu") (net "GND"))
 (segment (start 180.08 111.96) (end 183.76 115.64) (width 0.2) (layer "F.Cu") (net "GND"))
 (segment (start 123.46 97.8) (end 123.54 97.72) (width 0.2) (layer "F.Cu") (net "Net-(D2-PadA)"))
 (segment (start 117.04 97.8) (end 123.46 97.8) (width 0.2) (layer "F.Cu") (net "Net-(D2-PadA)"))
 (segment (start 130.1475 96.1925) (end 170.004714 96.1925) (width 0.2) (layer "F.Cu") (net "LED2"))
 (segment (start 173.6 99.787786) (end 173.6 100.4) (width 0.2) (layer "F.Cu") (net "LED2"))
 (segment (start 123.54 102.8) (end 130.1475 96.1925) (width 0.2) (layer "F.Cu") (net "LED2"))
 (segment (start 170.004714 96.1925) (end 173.6 99.787786) (width 0.2) (layer "F.Cu") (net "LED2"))
 (segment (start 162.08 97.8) (end 162.1 97.82) (width 0.2) (layer "F.Cu") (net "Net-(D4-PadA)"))
 (segment (start 155.2 97.8) (end 162.08 97.8) (width 0.2) (layer "F.Cu") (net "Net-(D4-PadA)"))
 (segment (start 162.1 106.68) (end 171.06 115.64) (width 0.2) (layer "B.Cu") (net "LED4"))
 (segment (start 162.1 102.9) (end 162.1 106.68) (width 0.2) (layer "B.Cu") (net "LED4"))
 (segment (start 172.01763 95.2) (end 176.14 99.32237) (width 0.2) (layer "F.Cu") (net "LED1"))
 (segment (start 176.14 99.32237) (end 176.14 100.4) (width 0.2) (layer "F.Cu") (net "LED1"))
 (segment (start 105.1 102.94) (end 112.84 95.2) (width 0.2) (layer "F.Cu") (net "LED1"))
 (segment (start 112.84 95.2) (end 172.01763 95.2) (width 0.2) (layer "F.Cu") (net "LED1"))
 (segment (start 104.96 98) (end 105.1 97.86) (width 0.2) (layer "F.Cu") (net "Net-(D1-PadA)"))
 (segment (start 97.7 98) (end 104.96 98) (width 0.2) (layer "F.Cu") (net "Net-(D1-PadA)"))
 (segment (start 172.538 115.663895) (end 166.901895 121.3) (width 0.2) (layer "B.Cu") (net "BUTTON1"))
 (segment (start 172.538 114.162) (end 172.538 115.663895) (width 0.2) (layer "B.Cu") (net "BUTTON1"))
 (segment (start 186.3 100.4) (end 172.538 114.162) (width 0.2) (layer "B.Cu") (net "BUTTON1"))
 (segment (start 166.901895 121.3) (end 109.262944 121.3) (width 0.2) (layer "B.Cu") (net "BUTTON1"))
 (segment (start 109.262944 121.3) (end 101.62 113.657056) (width 0.2) (layer "B.Cu") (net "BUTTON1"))
 (segment (start 101.62 113.657056) (end 101.62 109.42) (width 0.2) (layer "B.Cu") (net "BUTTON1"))
 (segment (start 120.66 109.42) (end 127.4 102.68) (width 0.2) (layer "B.Cu") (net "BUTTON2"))
 (segment (start 127.4 98.4) (end 129.6075 96.1925) (width 0.2) (layer "B.Cu") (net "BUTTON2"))
 (segment (start 129.6075 96.1925) (end 179.5525 96.1925) (width 0.2) (layer "B.Cu") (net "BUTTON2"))
 (segment (start 127.4 102.68) (end 127.4 98.4) (width 0.2) (layer "B.Cu") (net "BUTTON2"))
 (segment (start 179.5525 96.1925) (end 183.76 100.4) (width 0.2) (layer "B.Cu") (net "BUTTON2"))
 (segment (start 148.5 97.4) (end 149.3075 96.5925) (width 0.2) (layer "B.Cu") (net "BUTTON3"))
 (segment (start 148.5 100.68) (end 148.5 97.4) (width 0.2) (layer "B.Cu") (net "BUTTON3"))
 (segment (start 139.76 109.42) (end 148.5 100.68) (width 0.2) (layer "B.Cu") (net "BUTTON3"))
 (segment (start 177.4125 96.5925) (end 181.22 100.4) (width 0.2) (layer "B.Cu") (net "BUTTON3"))
 (segment (start 149.3075 96.5925) (end 177.4125 96.5925) (width 0.2) (layer "B.Cu") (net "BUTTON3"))
 (segment (start 177.618 101.462) (end 178.68 100.4) (width 0.2) (layer "B.Cu") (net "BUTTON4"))
 (segment (start 162.123786 101.462) (end 177.618 101.462) (width 0.2) (layer "B.Cu") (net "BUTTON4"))
 (segment (start 158.86 104.725786) (end 162.123786 101.462) (width 0.2) (layer "B.Cu") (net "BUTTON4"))
 (segment (start 158.86 109.42) (end 158.86 104.725786) (width 0.2) (layer "B.Cu") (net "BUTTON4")))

